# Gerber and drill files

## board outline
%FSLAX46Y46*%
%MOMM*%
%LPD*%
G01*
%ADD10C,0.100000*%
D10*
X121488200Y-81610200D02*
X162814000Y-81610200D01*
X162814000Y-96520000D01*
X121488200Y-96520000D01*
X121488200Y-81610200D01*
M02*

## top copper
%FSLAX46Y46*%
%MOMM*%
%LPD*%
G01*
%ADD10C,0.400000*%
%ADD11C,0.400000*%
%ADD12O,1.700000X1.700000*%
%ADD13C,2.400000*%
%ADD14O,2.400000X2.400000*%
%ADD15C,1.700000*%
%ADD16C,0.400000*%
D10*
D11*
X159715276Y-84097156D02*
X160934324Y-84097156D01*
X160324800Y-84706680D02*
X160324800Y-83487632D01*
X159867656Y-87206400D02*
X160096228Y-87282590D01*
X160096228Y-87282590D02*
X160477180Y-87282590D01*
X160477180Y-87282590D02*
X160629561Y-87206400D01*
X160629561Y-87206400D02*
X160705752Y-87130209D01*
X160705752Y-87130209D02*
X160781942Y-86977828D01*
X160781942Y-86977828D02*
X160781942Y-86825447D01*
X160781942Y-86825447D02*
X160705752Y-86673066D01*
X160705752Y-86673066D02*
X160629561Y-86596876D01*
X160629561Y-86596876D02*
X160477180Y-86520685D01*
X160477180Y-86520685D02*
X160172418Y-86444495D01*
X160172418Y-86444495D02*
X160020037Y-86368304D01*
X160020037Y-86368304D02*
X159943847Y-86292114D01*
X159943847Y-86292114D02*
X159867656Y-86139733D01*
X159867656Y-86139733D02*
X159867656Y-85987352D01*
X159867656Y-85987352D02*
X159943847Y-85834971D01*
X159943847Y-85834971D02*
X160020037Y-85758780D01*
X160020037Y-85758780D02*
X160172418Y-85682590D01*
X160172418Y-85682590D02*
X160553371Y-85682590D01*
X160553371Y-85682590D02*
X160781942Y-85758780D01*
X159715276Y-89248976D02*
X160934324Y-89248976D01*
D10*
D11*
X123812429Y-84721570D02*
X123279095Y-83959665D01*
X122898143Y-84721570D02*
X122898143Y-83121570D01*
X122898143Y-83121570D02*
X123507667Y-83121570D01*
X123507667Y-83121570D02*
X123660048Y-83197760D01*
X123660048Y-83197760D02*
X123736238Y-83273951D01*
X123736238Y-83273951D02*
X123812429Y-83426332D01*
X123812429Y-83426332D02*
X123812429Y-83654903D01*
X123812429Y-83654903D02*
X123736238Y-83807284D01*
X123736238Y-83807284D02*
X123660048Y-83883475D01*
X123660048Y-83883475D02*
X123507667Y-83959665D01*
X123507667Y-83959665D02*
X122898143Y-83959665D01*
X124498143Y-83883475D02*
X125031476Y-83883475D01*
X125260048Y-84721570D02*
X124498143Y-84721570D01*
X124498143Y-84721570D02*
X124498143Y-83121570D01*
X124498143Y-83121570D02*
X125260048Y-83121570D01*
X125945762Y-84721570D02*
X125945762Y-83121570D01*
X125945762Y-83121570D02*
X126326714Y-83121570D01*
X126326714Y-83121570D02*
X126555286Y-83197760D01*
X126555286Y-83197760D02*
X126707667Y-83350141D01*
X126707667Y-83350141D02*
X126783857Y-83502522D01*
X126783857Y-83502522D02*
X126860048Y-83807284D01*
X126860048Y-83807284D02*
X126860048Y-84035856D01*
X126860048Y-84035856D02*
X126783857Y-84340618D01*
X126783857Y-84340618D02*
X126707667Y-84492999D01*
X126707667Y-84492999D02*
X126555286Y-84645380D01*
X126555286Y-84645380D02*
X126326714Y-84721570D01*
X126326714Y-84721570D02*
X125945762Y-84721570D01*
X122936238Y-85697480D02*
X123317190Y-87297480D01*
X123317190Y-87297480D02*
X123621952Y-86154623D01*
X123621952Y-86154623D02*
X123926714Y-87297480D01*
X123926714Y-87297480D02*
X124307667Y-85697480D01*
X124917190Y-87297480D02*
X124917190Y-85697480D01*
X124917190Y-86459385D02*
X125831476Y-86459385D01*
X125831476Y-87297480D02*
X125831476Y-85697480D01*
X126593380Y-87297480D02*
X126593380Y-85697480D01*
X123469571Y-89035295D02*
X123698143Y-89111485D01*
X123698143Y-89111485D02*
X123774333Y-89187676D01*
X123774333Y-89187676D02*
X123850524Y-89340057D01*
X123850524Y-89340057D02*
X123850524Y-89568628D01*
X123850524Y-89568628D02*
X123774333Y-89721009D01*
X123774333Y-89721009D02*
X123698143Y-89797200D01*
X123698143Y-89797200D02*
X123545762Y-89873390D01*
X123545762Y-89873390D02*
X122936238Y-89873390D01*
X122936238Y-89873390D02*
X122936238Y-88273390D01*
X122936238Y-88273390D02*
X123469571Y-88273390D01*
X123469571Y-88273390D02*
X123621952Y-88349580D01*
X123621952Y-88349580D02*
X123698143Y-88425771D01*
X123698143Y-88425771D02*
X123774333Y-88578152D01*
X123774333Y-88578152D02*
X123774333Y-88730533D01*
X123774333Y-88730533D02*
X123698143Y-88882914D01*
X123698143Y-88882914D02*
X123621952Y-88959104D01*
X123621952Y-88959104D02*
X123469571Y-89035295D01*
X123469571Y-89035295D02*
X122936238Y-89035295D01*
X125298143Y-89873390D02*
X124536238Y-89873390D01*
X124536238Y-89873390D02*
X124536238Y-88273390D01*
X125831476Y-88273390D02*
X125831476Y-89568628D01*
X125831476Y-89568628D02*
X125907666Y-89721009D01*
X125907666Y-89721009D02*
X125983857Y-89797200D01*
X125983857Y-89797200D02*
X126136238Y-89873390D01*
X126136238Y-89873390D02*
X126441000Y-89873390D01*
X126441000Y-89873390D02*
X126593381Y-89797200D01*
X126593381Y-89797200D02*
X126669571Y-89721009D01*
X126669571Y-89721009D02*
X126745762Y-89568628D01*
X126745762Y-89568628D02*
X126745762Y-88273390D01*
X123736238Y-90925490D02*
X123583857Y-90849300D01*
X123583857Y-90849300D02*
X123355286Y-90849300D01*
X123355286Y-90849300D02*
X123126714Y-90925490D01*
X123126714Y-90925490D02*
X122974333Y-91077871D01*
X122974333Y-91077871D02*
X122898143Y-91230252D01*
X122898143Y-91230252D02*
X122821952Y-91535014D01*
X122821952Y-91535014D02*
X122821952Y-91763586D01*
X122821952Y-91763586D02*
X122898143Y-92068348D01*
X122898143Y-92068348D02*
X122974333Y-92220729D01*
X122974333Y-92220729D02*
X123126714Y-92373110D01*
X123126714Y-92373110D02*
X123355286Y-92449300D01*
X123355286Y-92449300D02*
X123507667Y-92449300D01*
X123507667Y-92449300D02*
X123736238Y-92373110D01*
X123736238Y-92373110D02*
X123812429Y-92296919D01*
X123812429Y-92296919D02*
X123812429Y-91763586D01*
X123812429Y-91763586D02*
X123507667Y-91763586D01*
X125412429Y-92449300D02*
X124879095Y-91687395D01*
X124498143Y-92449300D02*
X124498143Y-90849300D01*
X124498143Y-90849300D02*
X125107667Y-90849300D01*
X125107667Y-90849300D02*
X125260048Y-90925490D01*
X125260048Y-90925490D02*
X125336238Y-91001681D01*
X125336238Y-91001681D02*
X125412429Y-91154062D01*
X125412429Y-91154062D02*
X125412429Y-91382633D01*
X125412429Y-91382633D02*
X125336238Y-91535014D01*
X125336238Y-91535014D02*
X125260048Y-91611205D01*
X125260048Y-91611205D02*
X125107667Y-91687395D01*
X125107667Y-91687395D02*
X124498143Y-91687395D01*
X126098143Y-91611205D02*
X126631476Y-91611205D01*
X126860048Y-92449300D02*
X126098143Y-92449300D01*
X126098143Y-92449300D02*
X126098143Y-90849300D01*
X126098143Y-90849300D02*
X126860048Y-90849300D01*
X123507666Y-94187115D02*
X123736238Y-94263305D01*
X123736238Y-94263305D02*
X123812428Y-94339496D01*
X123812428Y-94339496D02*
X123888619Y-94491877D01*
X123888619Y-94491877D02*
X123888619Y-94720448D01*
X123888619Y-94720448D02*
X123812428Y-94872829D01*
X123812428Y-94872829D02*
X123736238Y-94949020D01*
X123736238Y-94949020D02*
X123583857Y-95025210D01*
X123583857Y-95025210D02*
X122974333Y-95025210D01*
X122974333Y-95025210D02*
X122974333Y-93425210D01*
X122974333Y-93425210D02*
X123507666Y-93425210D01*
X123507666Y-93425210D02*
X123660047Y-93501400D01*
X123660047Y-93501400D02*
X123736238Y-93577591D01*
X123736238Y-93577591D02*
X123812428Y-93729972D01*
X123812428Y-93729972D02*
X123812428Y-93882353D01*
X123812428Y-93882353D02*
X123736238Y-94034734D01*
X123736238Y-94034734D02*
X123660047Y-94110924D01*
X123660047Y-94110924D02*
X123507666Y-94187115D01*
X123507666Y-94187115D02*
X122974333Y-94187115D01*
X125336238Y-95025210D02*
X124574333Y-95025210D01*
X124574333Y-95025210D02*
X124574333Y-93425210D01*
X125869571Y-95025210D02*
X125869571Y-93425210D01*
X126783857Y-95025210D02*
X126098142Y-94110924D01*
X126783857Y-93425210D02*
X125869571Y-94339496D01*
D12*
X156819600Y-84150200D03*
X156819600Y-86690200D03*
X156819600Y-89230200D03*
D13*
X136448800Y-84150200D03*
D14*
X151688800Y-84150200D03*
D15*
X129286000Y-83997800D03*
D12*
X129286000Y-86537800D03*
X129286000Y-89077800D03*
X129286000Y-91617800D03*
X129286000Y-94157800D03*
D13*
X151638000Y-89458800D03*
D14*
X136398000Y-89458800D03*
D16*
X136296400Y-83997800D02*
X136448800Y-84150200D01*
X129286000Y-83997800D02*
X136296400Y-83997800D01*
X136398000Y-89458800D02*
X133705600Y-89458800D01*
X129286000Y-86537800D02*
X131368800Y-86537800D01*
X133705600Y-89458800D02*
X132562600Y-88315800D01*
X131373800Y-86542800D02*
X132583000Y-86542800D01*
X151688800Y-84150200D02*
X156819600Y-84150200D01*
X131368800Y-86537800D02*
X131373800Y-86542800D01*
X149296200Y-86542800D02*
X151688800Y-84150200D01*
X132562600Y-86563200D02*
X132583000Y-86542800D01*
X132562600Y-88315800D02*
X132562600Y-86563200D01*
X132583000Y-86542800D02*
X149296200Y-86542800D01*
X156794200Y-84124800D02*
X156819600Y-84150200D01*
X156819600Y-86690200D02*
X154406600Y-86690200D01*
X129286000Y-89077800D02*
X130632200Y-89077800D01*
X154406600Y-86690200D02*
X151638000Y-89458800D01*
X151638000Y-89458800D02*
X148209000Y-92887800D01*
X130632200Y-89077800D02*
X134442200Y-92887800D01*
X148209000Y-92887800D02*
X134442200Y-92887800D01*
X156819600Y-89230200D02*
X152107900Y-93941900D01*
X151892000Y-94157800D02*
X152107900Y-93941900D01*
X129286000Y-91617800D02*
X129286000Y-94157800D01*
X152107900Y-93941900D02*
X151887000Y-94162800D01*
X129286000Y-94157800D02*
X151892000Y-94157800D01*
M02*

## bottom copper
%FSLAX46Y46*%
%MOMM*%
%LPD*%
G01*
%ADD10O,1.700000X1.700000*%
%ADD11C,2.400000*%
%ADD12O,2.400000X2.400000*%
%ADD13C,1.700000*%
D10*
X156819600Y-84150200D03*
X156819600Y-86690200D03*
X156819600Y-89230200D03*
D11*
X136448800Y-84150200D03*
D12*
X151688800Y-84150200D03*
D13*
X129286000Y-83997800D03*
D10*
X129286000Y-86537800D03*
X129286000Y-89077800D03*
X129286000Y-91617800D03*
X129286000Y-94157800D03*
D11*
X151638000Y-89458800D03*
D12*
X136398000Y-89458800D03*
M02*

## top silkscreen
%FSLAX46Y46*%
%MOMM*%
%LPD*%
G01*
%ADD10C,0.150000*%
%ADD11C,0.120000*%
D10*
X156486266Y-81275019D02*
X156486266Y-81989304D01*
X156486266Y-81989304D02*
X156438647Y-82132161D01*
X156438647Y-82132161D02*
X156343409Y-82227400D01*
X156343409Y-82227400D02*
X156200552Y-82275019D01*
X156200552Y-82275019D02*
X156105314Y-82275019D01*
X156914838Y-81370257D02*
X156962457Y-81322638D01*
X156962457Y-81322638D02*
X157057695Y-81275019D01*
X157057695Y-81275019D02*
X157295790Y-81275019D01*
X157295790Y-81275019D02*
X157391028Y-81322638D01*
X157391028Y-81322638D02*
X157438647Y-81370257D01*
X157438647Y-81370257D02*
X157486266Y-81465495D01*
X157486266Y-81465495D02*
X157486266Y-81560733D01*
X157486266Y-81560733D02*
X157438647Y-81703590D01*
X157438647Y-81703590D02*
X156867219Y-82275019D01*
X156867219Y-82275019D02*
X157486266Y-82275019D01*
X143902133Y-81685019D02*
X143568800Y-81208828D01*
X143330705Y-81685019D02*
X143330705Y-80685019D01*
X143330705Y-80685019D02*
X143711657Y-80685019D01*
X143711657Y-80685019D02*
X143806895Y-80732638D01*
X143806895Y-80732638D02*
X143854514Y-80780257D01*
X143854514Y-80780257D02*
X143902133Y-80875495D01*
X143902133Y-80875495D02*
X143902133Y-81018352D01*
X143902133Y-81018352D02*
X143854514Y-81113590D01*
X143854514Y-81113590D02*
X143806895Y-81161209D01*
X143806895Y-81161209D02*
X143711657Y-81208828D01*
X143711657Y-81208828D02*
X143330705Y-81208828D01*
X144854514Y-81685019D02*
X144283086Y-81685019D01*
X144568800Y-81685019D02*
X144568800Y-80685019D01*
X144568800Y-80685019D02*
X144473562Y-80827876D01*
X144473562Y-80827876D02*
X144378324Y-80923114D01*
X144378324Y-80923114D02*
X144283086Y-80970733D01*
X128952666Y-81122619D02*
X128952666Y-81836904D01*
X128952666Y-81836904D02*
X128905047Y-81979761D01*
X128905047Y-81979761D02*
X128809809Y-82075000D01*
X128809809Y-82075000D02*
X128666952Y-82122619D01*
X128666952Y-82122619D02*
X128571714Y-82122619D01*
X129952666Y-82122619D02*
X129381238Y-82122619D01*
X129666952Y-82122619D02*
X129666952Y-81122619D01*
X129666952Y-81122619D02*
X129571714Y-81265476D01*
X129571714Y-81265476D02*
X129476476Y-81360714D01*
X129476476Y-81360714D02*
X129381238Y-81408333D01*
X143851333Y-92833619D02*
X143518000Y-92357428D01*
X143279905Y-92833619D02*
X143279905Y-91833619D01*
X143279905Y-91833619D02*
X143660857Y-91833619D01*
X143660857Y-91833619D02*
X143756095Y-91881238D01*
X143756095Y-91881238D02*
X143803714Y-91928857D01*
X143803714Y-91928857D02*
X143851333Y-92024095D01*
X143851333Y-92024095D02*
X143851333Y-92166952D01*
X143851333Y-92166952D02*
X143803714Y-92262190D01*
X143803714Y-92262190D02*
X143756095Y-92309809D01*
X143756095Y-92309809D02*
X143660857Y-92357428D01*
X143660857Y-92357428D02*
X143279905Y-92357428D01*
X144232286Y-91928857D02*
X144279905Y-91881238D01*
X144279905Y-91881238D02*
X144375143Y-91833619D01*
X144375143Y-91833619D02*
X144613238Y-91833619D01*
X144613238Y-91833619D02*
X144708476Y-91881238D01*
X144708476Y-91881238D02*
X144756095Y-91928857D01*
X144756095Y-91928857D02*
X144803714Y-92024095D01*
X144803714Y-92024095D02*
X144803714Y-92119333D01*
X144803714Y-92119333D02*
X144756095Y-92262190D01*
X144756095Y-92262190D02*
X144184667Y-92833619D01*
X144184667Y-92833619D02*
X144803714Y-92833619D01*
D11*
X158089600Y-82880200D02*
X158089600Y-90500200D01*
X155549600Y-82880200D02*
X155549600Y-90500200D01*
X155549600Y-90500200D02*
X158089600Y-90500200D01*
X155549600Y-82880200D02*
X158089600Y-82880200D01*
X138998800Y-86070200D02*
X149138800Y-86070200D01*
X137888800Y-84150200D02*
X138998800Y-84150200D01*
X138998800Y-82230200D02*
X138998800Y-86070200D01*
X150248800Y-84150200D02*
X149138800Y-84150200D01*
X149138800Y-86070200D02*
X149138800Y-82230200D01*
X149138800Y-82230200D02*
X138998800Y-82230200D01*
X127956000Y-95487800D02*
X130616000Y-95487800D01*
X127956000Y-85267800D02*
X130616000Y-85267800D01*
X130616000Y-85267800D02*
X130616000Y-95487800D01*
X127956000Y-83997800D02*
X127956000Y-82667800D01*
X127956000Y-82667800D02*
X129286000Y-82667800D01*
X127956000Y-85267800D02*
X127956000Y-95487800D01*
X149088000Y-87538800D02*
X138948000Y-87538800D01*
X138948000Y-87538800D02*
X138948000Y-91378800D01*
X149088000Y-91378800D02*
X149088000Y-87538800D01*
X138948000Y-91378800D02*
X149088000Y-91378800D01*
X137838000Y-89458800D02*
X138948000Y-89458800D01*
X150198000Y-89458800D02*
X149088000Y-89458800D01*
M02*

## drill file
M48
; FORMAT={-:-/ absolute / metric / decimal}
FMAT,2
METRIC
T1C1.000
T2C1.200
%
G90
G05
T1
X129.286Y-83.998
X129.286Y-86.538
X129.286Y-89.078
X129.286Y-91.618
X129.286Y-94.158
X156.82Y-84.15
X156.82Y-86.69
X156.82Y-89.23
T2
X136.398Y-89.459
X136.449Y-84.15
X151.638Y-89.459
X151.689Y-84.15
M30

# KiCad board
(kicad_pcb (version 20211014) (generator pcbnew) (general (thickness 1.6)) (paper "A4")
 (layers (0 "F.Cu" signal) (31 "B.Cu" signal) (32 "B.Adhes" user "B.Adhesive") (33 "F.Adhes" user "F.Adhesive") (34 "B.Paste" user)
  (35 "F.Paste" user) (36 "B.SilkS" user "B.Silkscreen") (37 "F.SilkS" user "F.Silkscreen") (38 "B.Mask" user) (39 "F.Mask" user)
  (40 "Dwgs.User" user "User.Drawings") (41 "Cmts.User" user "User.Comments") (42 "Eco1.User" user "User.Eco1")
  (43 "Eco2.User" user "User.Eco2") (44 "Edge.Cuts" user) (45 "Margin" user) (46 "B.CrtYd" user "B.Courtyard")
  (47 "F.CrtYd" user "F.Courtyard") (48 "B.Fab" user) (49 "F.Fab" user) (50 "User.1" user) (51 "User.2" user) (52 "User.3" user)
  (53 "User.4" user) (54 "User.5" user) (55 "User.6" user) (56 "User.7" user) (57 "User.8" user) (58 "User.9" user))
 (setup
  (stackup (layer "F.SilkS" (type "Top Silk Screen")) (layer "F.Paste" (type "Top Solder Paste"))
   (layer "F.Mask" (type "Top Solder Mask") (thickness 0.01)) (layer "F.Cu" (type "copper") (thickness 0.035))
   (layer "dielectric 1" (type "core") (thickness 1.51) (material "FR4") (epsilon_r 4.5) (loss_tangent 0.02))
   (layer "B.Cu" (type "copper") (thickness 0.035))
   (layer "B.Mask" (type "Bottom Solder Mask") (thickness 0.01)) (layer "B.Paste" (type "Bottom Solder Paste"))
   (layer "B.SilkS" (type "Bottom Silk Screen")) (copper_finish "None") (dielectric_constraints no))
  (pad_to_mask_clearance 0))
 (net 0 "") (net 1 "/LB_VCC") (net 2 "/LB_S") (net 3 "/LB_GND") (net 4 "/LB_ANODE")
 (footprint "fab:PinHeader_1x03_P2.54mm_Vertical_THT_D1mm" (layer "F.Cu") (at 156.8196 84.1502)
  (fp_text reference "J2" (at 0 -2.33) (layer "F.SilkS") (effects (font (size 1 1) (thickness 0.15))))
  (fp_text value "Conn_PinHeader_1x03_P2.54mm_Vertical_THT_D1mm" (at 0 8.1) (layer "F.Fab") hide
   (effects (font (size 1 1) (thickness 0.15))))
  (fp_line (start 1.27 -1.27) (end 1.27 6.35) (layer "F.SilkS") (width 0.12))
  (fp_line (start -1.27 -1.27) (end -1.27 6.35) (layer "F.SilkS") (width 0.12))
  (fp_line (start -1.27 6.35) (end 1.27 6.35) (layer "F.SilkS") (width 0.12))
  (fp_line (start -1.27 -1.27) (end 1.27 -1.27) (layer "F.SilkS") (width 0.12))
  (pad "1" thru_hole oval locked (at 0 0) (size 1.7 1.7) (drill 1) (layers *.Cu *.Mask) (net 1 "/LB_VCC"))
  (pad "2" thru_hole oval locked (at 0 2.54) (size 1.7 1.7) (drill 1) (layers *.Cu *.Mask) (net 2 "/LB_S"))
  (pad "3" thru_hole oval locked (at 0 5.08) (size 1.7 1.7) (drill 1) (layers *.Cu *.Mask) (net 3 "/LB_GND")))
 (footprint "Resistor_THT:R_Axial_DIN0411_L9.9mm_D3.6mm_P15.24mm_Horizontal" (layer "F.Cu") (at 136.4488 84.1502)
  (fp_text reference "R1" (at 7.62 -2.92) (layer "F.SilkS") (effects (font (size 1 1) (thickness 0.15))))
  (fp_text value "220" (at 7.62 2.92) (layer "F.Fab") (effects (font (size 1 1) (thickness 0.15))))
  (fp_line (start 2.55 1.92) (end 12.69 1.92) (layer "F.SilkS") (width 0.12))
  (fp_line (start 1.44 0) (end 2.55 0) (layer "F.SilkS") (width 0.12))
  (fp_line (start 2.55 -1.92) (end 2.55 1.92) (layer "F.SilkS") (width 0.12))
  (fp_line (start 13.8 0) (end 12.69 0) (layer "F.SilkS") (width 0.12))
  (fp_line (start 12.69 1.92) (end 12.69 -1.92) (layer "F.SilkS") (width 0.12))
  (fp_line (start 12.69 -1.92) (end 2.55 -1.92) (layer "F.SilkS") (width 0.12))
  (pad "1" thru_hole circle (at 0 0) (size 2.4 2.4) (drill 1.2) (layers *.Cu *.Mask) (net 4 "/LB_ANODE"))
  (pad "2" thru_hole oval (at 15.24 0) (size 2.4 2.4) (drill 1.2) (layers *.Cu *.Mask) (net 1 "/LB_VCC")))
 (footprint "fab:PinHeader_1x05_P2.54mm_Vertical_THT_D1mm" (layer "F.Cu") (at 129.286 83.9978)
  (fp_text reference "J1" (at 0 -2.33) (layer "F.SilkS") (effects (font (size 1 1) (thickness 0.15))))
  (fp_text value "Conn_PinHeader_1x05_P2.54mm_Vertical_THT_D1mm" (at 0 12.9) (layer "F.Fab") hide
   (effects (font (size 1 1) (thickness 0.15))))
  (fp_line (start -1.33 11.49) (end 1.33 11.49) (layer "F.SilkS") (width 0.12))
  (fp_line (start -1.33 1.27) (end 1.33 1.27) (layer "F.SilkS") (width 0.12))
  (fp_line (start 1.33 1.27) (end 1.33 11.49) (layer "F.SilkS") (width 0.12))
  (fp_line (start -1.33 0) (end -1.33 -1.33) (layer "F.SilkS") (width 0.12))
  (fp_line (start -1.33 -1.33) (end 0 -1.33) (layer "F.SilkS") (width 0.12))
  (fp_line (start -1.33 1.27) (end -1.33 11.49) (layer "F.SilkS") (width 0.12))
  (pad "1" thru_hole circle locked (at 0 0) (size 1.7 1.7) (drill 1) (layers *.Cu *.Mask) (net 4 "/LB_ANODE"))
  (pad "2" thru_hole oval locked (at 0 2.54) (size 1.7 1.7) (drill 1) (layers *.Cu *.Mask) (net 1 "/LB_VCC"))
  (pad "3" thru_hole oval locked (at 0 5.08) (size 1.7 1.7) (drill 1) (layers *.Cu *.Mask) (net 2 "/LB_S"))
  (pad "4" thru_hole oval locked (at 0 7.62) (size 1.7 1.7) (drill 1) (layers *.Cu *.Mask) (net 3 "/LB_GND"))
  (pad "5" thru_hole oval locked (at 0 10.16) (size 1.7 1.7) (drill 1) (layers *.Cu *.Mask) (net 3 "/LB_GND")))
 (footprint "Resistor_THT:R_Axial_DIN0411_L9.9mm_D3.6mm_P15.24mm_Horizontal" (layer "F.Cu") (at 151.638 89.4588 180)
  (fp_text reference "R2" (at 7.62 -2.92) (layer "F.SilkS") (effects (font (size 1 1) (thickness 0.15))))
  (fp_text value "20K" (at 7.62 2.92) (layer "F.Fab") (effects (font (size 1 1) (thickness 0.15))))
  (fp_line (start 2.55 1.92) (end 12.69 1.92) (layer "F.SilkS") (width 0.12))
  (fp_line (start 12.69 1.92) (end 12.69 -1.92) (layer "F.SilkS") (width 0.12))
  (fp_line (start 2.55 -1.92) (end 2.55 1.92) (layer "F.SilkS") (width 0.12))
  (fp_line (start 12.69 -1.92) (end 2.55 -1.92) (layer "F.SilkS") (width 0.12))
  (fp_line (start 13.8 0) (end 12.69 0) (layer "F.SilkS") (width 0.12))
  (fp_line (start 1.44 0) (end 2.55 0) (layer "F.SilkS") (width 0.12))
  (pad "1" thru_hole circle (at 0 0 180) (size 2.4 2.4) (drill 1.2) (layers *.Cu *.Mask) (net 2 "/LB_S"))
  (pad "2" thru_hole oval (at 15.24 0 180) (size 2.4 2.4) (drill 1.2) (layers *.Cu *.Mask) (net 1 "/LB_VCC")))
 (gr_rect (start 121.4882 81.6102) (end 162.814 96.52) (layer "Edge.Cuts") (width 0.1) (fill none))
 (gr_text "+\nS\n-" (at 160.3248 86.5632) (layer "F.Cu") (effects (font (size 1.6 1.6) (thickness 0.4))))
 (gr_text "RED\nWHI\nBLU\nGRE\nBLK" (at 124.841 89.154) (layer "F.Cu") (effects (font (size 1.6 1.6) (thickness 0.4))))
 (segment (start 136.2964 83.9978) (end 136.4488 84.1502) (width 0.4) (layer "F.Cu") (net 4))
 (segment (start 129.286 83.9978) (end 136.2964 83.9978) (width 0.4) (layer "F.Cu") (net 4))
 (segment (start 136.398 89.4588) (end 133.7056 89.4588) (width 0.4) (layer "F.Cu") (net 1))
 (segment (start 129.286 86.5378) (end 131.3688 86.5378) (width 0.4) (layer "F.Cu") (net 1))
 (segment (start 133.7056 89.4588) (end 132.5626 88.3158) (width 0.4) (layer "F.Cu") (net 1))
 (segment (start 131.3738 86.5428) (end 132.583 86.5428) (width 0.4) (layer "F.Cu") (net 1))
 (segment (start 151.6888 84.1502) (end 156.8196 84.1502) (width 0.4) (layer "F.Cu") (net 1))
 (segment (start 131.3688 86.5378) (end 131.3738 86.5428) (width 0.4) (layer "F.Cu") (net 1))
 (segment (start 149.2962 86.5428) (end 151.6888 84.1502) (width 0.4) (layer "F.Cu") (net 1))
 (segment (start 132.5626 86.5632) (end 132.583 86.5428) (width 0.4) (layer "F.Cu") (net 1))
 (segment (start 132.5626 88.3158) (end 132.5626 86.5632) (width 0.4) (layer "F.Cu") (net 1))
 (segment (start 132.583 86.5428) (end 149.2962 86.5428) (width 0.4) (layer "F.Cu") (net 1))
 (segment (start 156.7942 84.1248) (end 156.8196 84.1502) (width 0.4) (layer "F.Cu") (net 1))
 (segment (start 156.8196 86.6902) (end 154.4066 86.6902) (width 0.4) (layer "F.Cu") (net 2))
 (segment (start 129.286 89.0778) (end 130.6322 89.0778) (width 0.4) (layer "F.Cu") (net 2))
 (segment (start 154.4066 86.6902) (end 151.638 89.4588) (width 0.4) (layer "F.Cu") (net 2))
 (segment (start 151.638 89.4588) (end 148.209 92.8878) (width 0.4) (layer "F.Cu") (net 2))
 (segment (start 130.6322 89.0778) (end 134.4422 92.8878) (width 0.4) (layer "F.Cu") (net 2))
 (segment (start 148.209 92.8878) (end 134.4422 92.8878) (width 0.4) (layer "F.Cu") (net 2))
 (segment (start 156.8196 89.2302) (end 152.1079 93.9419) (width 0.4) (layer "F.Cu") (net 3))
 (segment (start 151.892 94.1578) (end 152.1079 93.9419) (width 0.4) (layer "F.Cu") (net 3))
 (segment (start 129.286 91.6178) (end 129.286 94.1578) (width 0.4) (layer "F.Cu") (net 3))
 (segment (start 152.1079 93.9419) (end 151.887 94.1628) (width 0.4) (layer "F.Cu") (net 3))
 (segment (start 129.286 94.1578) (end 151.892 94.1578) (width 0.4) (layer "F.Cu") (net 3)))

